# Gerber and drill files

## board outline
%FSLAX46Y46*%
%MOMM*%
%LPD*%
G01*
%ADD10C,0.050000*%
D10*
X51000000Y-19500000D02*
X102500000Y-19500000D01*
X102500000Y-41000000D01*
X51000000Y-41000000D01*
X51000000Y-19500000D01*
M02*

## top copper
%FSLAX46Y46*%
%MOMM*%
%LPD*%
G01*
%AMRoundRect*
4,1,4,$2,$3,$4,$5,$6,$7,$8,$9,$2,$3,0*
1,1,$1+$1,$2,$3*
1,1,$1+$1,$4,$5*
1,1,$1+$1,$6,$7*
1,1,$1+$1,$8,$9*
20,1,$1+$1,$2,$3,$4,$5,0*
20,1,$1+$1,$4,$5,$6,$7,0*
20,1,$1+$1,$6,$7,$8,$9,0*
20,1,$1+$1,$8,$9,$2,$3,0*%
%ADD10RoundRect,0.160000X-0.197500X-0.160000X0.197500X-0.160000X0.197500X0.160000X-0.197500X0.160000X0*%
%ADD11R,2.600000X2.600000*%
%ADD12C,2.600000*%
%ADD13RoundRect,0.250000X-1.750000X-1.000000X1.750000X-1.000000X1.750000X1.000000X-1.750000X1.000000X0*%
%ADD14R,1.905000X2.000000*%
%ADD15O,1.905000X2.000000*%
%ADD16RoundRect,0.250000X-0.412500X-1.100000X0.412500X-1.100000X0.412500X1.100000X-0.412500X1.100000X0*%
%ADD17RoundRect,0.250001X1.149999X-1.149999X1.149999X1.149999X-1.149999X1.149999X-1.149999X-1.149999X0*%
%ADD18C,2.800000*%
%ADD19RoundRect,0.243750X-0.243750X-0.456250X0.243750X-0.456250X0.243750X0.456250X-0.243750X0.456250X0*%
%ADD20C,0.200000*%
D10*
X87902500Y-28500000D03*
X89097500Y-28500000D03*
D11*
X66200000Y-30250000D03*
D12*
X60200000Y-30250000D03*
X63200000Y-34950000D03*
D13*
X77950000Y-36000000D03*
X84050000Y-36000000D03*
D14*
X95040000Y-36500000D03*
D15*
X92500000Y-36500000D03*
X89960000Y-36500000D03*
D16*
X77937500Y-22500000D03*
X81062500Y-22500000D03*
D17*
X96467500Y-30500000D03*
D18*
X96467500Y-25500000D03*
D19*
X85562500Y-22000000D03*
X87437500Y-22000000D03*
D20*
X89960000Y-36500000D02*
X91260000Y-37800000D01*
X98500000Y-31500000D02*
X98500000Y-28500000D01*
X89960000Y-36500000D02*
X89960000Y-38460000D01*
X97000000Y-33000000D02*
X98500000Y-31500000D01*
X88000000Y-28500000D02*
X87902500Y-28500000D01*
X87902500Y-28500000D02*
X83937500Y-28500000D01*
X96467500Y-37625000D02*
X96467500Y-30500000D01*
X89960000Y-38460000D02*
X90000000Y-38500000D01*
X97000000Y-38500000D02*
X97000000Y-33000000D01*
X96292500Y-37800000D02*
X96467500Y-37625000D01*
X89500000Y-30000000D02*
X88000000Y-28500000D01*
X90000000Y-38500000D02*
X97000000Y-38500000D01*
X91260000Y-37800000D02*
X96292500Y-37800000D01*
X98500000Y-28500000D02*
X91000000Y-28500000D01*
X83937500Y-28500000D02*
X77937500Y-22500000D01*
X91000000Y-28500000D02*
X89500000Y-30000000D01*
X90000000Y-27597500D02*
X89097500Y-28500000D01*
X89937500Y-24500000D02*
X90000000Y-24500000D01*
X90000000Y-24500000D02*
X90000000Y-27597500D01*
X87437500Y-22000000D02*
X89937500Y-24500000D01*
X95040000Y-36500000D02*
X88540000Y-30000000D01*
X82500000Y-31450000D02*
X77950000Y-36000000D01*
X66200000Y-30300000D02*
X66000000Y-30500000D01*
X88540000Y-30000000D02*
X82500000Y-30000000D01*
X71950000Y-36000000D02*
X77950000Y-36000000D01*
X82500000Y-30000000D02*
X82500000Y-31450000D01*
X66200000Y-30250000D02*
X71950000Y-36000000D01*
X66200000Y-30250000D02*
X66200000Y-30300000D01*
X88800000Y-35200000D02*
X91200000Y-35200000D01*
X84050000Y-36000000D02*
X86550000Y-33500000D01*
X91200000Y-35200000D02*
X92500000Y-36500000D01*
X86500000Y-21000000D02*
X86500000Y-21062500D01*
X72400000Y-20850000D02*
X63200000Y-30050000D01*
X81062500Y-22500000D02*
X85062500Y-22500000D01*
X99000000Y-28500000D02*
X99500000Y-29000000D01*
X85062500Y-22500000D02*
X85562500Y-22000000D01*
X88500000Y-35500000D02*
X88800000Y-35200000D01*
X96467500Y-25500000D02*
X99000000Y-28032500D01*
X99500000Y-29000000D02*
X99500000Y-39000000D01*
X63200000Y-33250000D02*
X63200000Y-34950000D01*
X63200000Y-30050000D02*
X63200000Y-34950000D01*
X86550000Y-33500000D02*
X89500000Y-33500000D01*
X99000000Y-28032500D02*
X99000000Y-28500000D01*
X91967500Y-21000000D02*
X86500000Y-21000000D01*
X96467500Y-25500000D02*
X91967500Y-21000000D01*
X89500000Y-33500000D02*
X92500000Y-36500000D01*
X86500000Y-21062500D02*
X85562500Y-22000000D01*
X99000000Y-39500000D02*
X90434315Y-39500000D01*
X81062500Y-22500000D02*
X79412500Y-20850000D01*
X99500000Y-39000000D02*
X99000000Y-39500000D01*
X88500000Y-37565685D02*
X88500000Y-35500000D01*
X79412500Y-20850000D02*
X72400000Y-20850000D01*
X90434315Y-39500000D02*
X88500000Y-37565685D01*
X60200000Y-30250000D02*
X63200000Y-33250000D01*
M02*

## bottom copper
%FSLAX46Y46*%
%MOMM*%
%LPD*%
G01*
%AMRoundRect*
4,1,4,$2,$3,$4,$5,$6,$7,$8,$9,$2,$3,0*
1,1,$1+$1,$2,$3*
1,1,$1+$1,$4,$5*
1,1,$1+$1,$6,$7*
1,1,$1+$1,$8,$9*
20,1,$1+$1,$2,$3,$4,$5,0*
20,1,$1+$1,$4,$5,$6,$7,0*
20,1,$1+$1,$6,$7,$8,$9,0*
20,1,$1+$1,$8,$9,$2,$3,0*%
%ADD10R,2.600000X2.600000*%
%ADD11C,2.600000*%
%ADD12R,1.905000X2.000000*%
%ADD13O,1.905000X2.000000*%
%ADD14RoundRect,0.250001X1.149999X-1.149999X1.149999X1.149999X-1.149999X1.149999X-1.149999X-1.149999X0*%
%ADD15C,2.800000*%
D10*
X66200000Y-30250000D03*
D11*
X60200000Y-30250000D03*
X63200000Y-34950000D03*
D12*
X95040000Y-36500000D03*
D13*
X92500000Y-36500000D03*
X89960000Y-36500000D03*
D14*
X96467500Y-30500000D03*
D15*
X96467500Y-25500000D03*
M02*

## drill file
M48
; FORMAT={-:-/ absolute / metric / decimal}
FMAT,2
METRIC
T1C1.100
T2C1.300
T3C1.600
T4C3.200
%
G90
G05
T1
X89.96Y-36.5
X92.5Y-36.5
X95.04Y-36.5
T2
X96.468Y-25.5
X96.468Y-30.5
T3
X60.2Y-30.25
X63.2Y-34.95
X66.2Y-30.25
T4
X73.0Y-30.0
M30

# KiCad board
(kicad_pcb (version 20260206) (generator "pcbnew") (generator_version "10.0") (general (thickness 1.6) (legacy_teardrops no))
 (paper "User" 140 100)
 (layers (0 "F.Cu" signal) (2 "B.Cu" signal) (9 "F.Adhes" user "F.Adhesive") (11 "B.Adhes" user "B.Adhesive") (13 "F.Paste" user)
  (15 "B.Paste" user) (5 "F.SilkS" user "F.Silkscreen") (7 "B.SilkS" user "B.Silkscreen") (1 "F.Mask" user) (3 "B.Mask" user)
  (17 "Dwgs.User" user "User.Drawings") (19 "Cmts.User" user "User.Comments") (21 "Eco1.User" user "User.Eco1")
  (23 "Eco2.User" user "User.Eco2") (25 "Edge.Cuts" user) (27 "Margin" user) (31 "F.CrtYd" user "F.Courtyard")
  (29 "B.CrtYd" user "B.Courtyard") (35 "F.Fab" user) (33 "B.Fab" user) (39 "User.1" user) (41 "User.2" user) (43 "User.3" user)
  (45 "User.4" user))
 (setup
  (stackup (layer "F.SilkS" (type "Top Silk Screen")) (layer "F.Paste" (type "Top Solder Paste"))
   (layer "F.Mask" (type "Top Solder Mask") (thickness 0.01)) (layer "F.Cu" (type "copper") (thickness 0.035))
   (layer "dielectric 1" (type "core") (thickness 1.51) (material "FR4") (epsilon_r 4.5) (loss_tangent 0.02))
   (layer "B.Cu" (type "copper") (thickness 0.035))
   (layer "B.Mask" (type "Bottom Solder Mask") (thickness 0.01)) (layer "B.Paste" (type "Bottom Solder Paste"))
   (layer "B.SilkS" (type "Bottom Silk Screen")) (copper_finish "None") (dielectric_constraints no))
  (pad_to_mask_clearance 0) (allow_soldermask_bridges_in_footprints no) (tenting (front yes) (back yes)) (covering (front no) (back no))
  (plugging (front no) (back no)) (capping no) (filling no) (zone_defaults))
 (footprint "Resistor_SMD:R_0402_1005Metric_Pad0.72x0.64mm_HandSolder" (layer "F.Cu") (at 88.5 28.5)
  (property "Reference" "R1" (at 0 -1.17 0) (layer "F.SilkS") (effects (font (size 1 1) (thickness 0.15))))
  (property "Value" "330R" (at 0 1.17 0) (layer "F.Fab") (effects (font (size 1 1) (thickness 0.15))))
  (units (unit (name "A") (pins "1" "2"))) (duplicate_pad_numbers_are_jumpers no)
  (pad "1" smd roundrect (at -0.5975 0) (size 0.715 0.64) (layers "F.Cu" "F.Mask" "F.Paste") (roundrect_rratio 0.25) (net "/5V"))
  (pad "2" smd roundrect (at 0.5975 0) (size 0.715 0.64) (layers "F.Cu" "F.Mask" "F.Paste") (roundrect_rratio 0.25) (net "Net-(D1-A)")))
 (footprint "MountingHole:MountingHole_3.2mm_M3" (layer "F.Cu") (at 73 30)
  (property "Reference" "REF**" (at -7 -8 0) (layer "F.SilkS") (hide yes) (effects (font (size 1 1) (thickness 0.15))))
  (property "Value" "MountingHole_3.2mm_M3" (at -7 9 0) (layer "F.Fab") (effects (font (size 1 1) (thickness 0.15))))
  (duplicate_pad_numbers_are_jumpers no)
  (pad "" np_thru_hole circle (at 0 0) (size 3.2 3.2) (drill 3.2) (layers "*.Cu" "*.Mask")))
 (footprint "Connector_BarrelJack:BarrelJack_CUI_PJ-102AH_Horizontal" (layer "F.Cu") (at 66.2 30.25 -90)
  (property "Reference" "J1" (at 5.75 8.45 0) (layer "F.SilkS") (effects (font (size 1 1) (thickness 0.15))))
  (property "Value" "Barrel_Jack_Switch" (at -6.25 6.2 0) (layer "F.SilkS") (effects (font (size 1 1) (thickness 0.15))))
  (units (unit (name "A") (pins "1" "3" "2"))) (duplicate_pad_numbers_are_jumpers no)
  (pad "1" thru_hole rect (at 0 0 270) (size 2.6 2.6) (drill 1.6) (layers "*.Cu" "*.Mask") (remove_unused_layers no) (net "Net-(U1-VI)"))
  (pad "2" thru_hole circle (at 0 6 270) (size 2.6 2.6) (drill 1.6) (layers "*.Cu" "*.Mask") (remove_unused_layers no) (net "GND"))
  (pad "3" thru_hole circle (at 4.7 3 270) (size 2.6 2.6) (drill 1.6) (layers "*.Cu" "*.Mask") (remove_unused_layers no) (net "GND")))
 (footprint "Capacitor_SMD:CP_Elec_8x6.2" (layer "F.Cu") (at 81 36)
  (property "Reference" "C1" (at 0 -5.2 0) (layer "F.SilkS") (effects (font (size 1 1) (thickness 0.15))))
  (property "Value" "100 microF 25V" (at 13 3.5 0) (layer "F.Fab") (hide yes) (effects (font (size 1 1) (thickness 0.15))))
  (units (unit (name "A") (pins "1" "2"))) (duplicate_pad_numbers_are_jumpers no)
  (pad "1" smd roundrect (at -3.05 0) (size 4 2.5) (layers "F.Cu" "F.Mask" "F.Paste") (roundrect_rratio 0.1) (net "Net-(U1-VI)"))
  (pad "2" smd roundrect (at 3.05 0) (size 4 2.5) (layers "F.Cu" "F.Mask" "F.Paste") (roundrect_rratio 0.1) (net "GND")))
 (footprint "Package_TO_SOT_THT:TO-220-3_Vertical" (layer "F.Cu") (at 95.04 36.5 180)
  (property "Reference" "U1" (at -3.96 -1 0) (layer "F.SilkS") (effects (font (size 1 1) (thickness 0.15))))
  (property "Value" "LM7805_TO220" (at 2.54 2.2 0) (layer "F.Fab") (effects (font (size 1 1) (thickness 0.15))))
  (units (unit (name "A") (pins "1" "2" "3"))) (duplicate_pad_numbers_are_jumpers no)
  (pad "1" thru_hole rect (at 0 0 180) (size 1.905 2) (drill 1.1) (layers "*.Cu" "*.Mask") (remove_unused_layers no) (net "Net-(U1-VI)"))
  (pad "2" thru_hole oval (at 2.54 0 180) (size 1.905 2) (drill 1.1) (layers "*.Cu" "*.Mask") (remove_unused_layers no) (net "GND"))
  (pad "3" thru_hole oval (at 5.08 0 180) (size 1.905 2) (drill 1.1) (layers "*.Cu" "*.Mask") (remove_unused_layers no) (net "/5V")))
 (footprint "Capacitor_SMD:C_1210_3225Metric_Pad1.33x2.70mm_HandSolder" (layer "F.Cu") (at 79.5 22.5)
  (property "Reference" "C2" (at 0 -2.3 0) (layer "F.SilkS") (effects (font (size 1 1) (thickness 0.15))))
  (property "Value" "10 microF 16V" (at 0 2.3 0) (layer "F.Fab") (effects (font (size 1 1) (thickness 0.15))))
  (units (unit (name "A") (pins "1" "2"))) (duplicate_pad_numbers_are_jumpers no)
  (pad "1" smd roundrect (at -1.5625 0) (size 1.325 2.7) (layers "F.Cu" "F.Mask" "F.Paste") (roundrect_rratio 0.188679) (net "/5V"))
  (pad "2" smd roundrect (at 1.5625 0) (size 1.325 2.7) (layers "F.Cu" "F.Mask" "F.Paste") (roundrect_rratio 0.188679) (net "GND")))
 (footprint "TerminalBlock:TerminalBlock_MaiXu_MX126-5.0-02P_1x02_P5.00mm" (layer "F.Cu") (at 96.4675 30.5 90)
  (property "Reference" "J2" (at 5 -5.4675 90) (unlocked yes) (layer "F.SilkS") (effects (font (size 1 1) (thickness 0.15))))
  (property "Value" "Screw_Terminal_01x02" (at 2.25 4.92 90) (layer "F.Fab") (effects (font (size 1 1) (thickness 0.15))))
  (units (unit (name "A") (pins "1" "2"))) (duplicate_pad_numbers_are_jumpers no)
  (pad "1" thru_hole roundrect (at 0 0 90) (size 2.8 2.8) (drill 1.3) (layers "*.Cu" "*.Mask") (remove_unused_layers no)
   (roundrect_rratio 0.089286) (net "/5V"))
  (pad "2" thru_hole circle (at 5 0 90) (size 2.8 2.8) (drill 1.3) (layers "*.Cu" "*.Mask") (remove_unused_layers no) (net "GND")))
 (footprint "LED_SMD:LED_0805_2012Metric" (layer "F.Cu") (at 86.5 22)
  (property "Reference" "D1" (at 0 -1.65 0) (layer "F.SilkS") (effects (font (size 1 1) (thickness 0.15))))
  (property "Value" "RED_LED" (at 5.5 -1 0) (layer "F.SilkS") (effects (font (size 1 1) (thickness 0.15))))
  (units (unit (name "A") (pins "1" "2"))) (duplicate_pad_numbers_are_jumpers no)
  (pad "1" smd roundrect (at -0.9375 0) (size 0.975 1.4) (layers "F.Cu" "F.Mask" "F.Paste") (roundrect_rratio 0.25) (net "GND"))
  (pad "2" smd roundrect (at 0.9375 0) (size 0.975 1.4) (layers "F.Cu" "F.Mask" "F.Paste") (roundrect_rratio 0.25) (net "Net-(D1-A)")))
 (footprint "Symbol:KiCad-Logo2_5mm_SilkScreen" (layer "B.Cu") (at 88.5 31.5 180)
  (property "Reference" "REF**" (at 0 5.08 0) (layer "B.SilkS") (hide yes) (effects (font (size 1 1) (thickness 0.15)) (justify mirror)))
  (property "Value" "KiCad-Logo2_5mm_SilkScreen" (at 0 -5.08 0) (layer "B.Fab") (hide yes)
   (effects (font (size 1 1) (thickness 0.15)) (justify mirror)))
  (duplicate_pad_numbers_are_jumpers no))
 (gr_rect (start 51 19.5) (end 102.5 41) (stroke (width 0.05) (type solid)) (fill no) (layer "Edge.Cuts"))
 (segment (start 89.96 36.5) (end 91.26 37.8) (width 0.2) (layer "F.Cu") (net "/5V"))
 (segment (start 98.5 31.5) (end 98.5 28.5) (width 0.2) (layer "F.Cu") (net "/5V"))
 (segment (start 89.96 36.5) (end 89.96 38.46) (width 0.2) (layer "F.Cu") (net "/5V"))
 (segment (start 97 33) (end 98.5 31.5) (width 0.2) (layer "F.Cu") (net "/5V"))
 (segment (start 88 28.5) (end 87.9025 28.5) (width 0.2) (layer "F.Cu") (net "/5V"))
 (segment (start 87.9025 28.5) (end 83.9375 28.5) (width 0.2) (layer "F.Cu") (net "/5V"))
 (segment (start 96.4675 37.625) (end 96.4675 30.5) (width 0.2) (layer "F.Cu") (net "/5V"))
 (segment (start 89.96 38.46) (end 90 38.5) (width 0.2) (layer "F.Cu") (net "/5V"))
 (segment (start 97 38.5) (end 97 33) (width 0.2) (layer "F.Cu") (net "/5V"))
 (segment (start 96.2925 37.8) (end 96.4675 37.625) (width 0.2) (layer "F.Cu") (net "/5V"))
 (segment (start 89.5 30) (end 88 28.5) (width 0.2) (layer "F.Cu") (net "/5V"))
 (segment (start 90 38.5) (end 97 38.5) (width 0.2) (layer "F.Cu") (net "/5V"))
 (segment (start 91.26 37.8) (end 96.2925 37.8) (width 0.2) (layer "F.Cu") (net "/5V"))
 (segment (start 98.5 28.5) (end 91 28.5) (width 0.2) (layer "F.Cu") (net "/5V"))
 (segment (start 83.9375 28.5) (end 77.9375 22.5) (width 0.2) (layer "F.Cu") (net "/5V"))
 (segment (start 91 28.5) (end 89.5 30) (width 0.2) (layer "F.Cu") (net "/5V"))
 (segment (start 90 27.5975) (end 89.0975 28.5) (width 0.2) (layer "F.Cu") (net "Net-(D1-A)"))
 (segment (start 89.9375 24.5) (end 90 24.5) (width 0.2) (layer "F.Cu") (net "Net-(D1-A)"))
 (segment (start 90 24.5) (end 90 27.5975) (width 0.2) (layer "F.Cu") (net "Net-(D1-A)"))
 (segment (start 87.4375 22) (end 89.9375 24.5) (width 0.2) (layer "F.Cu") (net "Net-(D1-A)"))
 (segment (start 95.04 36.5) (end 88.54 30) (width 0.2) (layer "F.Cu") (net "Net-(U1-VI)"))
 (segment (start 82.5 31.45) (end 77.95 36) (width 0.2) (layer "F.Cu") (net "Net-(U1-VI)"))
 (segment (start 66.2 30.3) (end 66 30.5) (width 0.2) (layer "F.Cu") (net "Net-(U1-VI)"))
 (segment (start 88.54 30) (end 82.5 30) (width 0.2) (layer "F.Cu") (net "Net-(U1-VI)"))
 (segment (start 71.95 36) (end 77.95 36) (width 0.2) (layer "F.Cu") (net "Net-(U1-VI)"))
 (segment (start 82.5 30) (end 82.5 31.45) (width 0.2) (layer "F.Cu") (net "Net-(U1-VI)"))
 (segment (start 66.2 30.25) (end 71.95 36) (width 0.2) (layer "F.Cu") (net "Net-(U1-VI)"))
 (segment (start 66.2 30.25) (end 66.2 30.3) (width 0.2) (layer "F.Cu") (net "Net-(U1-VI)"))
 (segment (start 88.8 35.2) (end 91.2 35.2) (width 0.2) (layer "F.Cu") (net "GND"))
 (segment (start 84.05 36) (end 86.55 33.5) (width 0.2) (layer "F.Cu") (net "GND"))
 (segment (start 91.2 35.2) (end 92.5 36.5) (width 0.2) (layer "F.Cu") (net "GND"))
 (segment (start 86.5 21) (end 86.5 21.0625) (width 0.2) (layer "F.Cu") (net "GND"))
 (segment (start 72.4 20.85) (end 63.2 30.05) (width 0.2) (layer "F.Cu") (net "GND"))
 (segment (start 81.0625 22.5) (end 85.0625 22.5) (width 0.2) (layer "F.Cu") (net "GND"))
 (segment (start 99 28.5) (end 99.5 29) (width 0.2) (layer "F.Cu") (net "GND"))
 (segment (start 85.0625 22.5) (end 85.5625 22) (width 0.2) (layer "F.Cu") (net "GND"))
 (segment (start 88.5 35.5) (end 88.8 35.2) (width 0.2) (layer "F.Cu") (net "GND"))
 (segment (start 96.4675 25.5) (end 99 28.0325) (width 0.2) (layer "F.Cu") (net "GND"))
 (segment (start 99.5 29) (end 99.5 39) (width 0.2) (layer "F.Cu") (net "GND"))
 (segment (start 63.2 33.25) (end 63.2 34.95) (width 0.2) (layer "F.Cu") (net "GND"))
 (segment (start 63.2 30.05) (end 63.2 34.95) (width 0.2) (layer "F.Cu") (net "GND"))
 (segment (start 86.55 33.5) (end 89.5 33.5) (width 0.2) (layer "F.Cu") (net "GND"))
 (segment (start 99 28.0325) (end 99 28.5) (width 0.2) (layer "F.Cu") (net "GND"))
 (segment (start 91.9675 21) (end 86.5 21) (width 0.2) (layer "F.Cu") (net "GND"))
 (segment (start 96.4675 25.5) (end 91.9675 21) (width 0.2) (layer "F.Cu") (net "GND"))
 (segment (start 89.5 33.5) (end 92.5 36.5) (width 0.2) (layer "F.Cu") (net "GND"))
 (segment (start 86.5 21.0625) (end 85.5625 22) (width 0.2) (layer "F.Cu") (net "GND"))
 (segment (start 99 39.5) (end 90.434315 39.5) (width 0.2) (layer "F.Cu") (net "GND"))
 (segment (start 81.0625 22.5) (end 79.4125 20.85) (width 0.2) (layer "F.Cu") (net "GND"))
 (segment (start 99.5 39) (end 99 39.5) (width 0.2) (layer "F.Cu") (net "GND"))
 (segment (start 88.5 37.565685) (end 88.5 35.5) (width 0.2) (layer "F.Cu") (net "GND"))
 (segment (start 79.4125 20.85) (end 72.4 20.85) (width 0.2) (layer "F.Cu") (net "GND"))
 (segment (start 90.434315 39.5) (end 88.5 37.565685) (width 0.2) (layer "F.Cu") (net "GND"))
 (segment (start 60.2 30.25) (end 63.2 33.25) (width 0.2) (layer "F.Cu") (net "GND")))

